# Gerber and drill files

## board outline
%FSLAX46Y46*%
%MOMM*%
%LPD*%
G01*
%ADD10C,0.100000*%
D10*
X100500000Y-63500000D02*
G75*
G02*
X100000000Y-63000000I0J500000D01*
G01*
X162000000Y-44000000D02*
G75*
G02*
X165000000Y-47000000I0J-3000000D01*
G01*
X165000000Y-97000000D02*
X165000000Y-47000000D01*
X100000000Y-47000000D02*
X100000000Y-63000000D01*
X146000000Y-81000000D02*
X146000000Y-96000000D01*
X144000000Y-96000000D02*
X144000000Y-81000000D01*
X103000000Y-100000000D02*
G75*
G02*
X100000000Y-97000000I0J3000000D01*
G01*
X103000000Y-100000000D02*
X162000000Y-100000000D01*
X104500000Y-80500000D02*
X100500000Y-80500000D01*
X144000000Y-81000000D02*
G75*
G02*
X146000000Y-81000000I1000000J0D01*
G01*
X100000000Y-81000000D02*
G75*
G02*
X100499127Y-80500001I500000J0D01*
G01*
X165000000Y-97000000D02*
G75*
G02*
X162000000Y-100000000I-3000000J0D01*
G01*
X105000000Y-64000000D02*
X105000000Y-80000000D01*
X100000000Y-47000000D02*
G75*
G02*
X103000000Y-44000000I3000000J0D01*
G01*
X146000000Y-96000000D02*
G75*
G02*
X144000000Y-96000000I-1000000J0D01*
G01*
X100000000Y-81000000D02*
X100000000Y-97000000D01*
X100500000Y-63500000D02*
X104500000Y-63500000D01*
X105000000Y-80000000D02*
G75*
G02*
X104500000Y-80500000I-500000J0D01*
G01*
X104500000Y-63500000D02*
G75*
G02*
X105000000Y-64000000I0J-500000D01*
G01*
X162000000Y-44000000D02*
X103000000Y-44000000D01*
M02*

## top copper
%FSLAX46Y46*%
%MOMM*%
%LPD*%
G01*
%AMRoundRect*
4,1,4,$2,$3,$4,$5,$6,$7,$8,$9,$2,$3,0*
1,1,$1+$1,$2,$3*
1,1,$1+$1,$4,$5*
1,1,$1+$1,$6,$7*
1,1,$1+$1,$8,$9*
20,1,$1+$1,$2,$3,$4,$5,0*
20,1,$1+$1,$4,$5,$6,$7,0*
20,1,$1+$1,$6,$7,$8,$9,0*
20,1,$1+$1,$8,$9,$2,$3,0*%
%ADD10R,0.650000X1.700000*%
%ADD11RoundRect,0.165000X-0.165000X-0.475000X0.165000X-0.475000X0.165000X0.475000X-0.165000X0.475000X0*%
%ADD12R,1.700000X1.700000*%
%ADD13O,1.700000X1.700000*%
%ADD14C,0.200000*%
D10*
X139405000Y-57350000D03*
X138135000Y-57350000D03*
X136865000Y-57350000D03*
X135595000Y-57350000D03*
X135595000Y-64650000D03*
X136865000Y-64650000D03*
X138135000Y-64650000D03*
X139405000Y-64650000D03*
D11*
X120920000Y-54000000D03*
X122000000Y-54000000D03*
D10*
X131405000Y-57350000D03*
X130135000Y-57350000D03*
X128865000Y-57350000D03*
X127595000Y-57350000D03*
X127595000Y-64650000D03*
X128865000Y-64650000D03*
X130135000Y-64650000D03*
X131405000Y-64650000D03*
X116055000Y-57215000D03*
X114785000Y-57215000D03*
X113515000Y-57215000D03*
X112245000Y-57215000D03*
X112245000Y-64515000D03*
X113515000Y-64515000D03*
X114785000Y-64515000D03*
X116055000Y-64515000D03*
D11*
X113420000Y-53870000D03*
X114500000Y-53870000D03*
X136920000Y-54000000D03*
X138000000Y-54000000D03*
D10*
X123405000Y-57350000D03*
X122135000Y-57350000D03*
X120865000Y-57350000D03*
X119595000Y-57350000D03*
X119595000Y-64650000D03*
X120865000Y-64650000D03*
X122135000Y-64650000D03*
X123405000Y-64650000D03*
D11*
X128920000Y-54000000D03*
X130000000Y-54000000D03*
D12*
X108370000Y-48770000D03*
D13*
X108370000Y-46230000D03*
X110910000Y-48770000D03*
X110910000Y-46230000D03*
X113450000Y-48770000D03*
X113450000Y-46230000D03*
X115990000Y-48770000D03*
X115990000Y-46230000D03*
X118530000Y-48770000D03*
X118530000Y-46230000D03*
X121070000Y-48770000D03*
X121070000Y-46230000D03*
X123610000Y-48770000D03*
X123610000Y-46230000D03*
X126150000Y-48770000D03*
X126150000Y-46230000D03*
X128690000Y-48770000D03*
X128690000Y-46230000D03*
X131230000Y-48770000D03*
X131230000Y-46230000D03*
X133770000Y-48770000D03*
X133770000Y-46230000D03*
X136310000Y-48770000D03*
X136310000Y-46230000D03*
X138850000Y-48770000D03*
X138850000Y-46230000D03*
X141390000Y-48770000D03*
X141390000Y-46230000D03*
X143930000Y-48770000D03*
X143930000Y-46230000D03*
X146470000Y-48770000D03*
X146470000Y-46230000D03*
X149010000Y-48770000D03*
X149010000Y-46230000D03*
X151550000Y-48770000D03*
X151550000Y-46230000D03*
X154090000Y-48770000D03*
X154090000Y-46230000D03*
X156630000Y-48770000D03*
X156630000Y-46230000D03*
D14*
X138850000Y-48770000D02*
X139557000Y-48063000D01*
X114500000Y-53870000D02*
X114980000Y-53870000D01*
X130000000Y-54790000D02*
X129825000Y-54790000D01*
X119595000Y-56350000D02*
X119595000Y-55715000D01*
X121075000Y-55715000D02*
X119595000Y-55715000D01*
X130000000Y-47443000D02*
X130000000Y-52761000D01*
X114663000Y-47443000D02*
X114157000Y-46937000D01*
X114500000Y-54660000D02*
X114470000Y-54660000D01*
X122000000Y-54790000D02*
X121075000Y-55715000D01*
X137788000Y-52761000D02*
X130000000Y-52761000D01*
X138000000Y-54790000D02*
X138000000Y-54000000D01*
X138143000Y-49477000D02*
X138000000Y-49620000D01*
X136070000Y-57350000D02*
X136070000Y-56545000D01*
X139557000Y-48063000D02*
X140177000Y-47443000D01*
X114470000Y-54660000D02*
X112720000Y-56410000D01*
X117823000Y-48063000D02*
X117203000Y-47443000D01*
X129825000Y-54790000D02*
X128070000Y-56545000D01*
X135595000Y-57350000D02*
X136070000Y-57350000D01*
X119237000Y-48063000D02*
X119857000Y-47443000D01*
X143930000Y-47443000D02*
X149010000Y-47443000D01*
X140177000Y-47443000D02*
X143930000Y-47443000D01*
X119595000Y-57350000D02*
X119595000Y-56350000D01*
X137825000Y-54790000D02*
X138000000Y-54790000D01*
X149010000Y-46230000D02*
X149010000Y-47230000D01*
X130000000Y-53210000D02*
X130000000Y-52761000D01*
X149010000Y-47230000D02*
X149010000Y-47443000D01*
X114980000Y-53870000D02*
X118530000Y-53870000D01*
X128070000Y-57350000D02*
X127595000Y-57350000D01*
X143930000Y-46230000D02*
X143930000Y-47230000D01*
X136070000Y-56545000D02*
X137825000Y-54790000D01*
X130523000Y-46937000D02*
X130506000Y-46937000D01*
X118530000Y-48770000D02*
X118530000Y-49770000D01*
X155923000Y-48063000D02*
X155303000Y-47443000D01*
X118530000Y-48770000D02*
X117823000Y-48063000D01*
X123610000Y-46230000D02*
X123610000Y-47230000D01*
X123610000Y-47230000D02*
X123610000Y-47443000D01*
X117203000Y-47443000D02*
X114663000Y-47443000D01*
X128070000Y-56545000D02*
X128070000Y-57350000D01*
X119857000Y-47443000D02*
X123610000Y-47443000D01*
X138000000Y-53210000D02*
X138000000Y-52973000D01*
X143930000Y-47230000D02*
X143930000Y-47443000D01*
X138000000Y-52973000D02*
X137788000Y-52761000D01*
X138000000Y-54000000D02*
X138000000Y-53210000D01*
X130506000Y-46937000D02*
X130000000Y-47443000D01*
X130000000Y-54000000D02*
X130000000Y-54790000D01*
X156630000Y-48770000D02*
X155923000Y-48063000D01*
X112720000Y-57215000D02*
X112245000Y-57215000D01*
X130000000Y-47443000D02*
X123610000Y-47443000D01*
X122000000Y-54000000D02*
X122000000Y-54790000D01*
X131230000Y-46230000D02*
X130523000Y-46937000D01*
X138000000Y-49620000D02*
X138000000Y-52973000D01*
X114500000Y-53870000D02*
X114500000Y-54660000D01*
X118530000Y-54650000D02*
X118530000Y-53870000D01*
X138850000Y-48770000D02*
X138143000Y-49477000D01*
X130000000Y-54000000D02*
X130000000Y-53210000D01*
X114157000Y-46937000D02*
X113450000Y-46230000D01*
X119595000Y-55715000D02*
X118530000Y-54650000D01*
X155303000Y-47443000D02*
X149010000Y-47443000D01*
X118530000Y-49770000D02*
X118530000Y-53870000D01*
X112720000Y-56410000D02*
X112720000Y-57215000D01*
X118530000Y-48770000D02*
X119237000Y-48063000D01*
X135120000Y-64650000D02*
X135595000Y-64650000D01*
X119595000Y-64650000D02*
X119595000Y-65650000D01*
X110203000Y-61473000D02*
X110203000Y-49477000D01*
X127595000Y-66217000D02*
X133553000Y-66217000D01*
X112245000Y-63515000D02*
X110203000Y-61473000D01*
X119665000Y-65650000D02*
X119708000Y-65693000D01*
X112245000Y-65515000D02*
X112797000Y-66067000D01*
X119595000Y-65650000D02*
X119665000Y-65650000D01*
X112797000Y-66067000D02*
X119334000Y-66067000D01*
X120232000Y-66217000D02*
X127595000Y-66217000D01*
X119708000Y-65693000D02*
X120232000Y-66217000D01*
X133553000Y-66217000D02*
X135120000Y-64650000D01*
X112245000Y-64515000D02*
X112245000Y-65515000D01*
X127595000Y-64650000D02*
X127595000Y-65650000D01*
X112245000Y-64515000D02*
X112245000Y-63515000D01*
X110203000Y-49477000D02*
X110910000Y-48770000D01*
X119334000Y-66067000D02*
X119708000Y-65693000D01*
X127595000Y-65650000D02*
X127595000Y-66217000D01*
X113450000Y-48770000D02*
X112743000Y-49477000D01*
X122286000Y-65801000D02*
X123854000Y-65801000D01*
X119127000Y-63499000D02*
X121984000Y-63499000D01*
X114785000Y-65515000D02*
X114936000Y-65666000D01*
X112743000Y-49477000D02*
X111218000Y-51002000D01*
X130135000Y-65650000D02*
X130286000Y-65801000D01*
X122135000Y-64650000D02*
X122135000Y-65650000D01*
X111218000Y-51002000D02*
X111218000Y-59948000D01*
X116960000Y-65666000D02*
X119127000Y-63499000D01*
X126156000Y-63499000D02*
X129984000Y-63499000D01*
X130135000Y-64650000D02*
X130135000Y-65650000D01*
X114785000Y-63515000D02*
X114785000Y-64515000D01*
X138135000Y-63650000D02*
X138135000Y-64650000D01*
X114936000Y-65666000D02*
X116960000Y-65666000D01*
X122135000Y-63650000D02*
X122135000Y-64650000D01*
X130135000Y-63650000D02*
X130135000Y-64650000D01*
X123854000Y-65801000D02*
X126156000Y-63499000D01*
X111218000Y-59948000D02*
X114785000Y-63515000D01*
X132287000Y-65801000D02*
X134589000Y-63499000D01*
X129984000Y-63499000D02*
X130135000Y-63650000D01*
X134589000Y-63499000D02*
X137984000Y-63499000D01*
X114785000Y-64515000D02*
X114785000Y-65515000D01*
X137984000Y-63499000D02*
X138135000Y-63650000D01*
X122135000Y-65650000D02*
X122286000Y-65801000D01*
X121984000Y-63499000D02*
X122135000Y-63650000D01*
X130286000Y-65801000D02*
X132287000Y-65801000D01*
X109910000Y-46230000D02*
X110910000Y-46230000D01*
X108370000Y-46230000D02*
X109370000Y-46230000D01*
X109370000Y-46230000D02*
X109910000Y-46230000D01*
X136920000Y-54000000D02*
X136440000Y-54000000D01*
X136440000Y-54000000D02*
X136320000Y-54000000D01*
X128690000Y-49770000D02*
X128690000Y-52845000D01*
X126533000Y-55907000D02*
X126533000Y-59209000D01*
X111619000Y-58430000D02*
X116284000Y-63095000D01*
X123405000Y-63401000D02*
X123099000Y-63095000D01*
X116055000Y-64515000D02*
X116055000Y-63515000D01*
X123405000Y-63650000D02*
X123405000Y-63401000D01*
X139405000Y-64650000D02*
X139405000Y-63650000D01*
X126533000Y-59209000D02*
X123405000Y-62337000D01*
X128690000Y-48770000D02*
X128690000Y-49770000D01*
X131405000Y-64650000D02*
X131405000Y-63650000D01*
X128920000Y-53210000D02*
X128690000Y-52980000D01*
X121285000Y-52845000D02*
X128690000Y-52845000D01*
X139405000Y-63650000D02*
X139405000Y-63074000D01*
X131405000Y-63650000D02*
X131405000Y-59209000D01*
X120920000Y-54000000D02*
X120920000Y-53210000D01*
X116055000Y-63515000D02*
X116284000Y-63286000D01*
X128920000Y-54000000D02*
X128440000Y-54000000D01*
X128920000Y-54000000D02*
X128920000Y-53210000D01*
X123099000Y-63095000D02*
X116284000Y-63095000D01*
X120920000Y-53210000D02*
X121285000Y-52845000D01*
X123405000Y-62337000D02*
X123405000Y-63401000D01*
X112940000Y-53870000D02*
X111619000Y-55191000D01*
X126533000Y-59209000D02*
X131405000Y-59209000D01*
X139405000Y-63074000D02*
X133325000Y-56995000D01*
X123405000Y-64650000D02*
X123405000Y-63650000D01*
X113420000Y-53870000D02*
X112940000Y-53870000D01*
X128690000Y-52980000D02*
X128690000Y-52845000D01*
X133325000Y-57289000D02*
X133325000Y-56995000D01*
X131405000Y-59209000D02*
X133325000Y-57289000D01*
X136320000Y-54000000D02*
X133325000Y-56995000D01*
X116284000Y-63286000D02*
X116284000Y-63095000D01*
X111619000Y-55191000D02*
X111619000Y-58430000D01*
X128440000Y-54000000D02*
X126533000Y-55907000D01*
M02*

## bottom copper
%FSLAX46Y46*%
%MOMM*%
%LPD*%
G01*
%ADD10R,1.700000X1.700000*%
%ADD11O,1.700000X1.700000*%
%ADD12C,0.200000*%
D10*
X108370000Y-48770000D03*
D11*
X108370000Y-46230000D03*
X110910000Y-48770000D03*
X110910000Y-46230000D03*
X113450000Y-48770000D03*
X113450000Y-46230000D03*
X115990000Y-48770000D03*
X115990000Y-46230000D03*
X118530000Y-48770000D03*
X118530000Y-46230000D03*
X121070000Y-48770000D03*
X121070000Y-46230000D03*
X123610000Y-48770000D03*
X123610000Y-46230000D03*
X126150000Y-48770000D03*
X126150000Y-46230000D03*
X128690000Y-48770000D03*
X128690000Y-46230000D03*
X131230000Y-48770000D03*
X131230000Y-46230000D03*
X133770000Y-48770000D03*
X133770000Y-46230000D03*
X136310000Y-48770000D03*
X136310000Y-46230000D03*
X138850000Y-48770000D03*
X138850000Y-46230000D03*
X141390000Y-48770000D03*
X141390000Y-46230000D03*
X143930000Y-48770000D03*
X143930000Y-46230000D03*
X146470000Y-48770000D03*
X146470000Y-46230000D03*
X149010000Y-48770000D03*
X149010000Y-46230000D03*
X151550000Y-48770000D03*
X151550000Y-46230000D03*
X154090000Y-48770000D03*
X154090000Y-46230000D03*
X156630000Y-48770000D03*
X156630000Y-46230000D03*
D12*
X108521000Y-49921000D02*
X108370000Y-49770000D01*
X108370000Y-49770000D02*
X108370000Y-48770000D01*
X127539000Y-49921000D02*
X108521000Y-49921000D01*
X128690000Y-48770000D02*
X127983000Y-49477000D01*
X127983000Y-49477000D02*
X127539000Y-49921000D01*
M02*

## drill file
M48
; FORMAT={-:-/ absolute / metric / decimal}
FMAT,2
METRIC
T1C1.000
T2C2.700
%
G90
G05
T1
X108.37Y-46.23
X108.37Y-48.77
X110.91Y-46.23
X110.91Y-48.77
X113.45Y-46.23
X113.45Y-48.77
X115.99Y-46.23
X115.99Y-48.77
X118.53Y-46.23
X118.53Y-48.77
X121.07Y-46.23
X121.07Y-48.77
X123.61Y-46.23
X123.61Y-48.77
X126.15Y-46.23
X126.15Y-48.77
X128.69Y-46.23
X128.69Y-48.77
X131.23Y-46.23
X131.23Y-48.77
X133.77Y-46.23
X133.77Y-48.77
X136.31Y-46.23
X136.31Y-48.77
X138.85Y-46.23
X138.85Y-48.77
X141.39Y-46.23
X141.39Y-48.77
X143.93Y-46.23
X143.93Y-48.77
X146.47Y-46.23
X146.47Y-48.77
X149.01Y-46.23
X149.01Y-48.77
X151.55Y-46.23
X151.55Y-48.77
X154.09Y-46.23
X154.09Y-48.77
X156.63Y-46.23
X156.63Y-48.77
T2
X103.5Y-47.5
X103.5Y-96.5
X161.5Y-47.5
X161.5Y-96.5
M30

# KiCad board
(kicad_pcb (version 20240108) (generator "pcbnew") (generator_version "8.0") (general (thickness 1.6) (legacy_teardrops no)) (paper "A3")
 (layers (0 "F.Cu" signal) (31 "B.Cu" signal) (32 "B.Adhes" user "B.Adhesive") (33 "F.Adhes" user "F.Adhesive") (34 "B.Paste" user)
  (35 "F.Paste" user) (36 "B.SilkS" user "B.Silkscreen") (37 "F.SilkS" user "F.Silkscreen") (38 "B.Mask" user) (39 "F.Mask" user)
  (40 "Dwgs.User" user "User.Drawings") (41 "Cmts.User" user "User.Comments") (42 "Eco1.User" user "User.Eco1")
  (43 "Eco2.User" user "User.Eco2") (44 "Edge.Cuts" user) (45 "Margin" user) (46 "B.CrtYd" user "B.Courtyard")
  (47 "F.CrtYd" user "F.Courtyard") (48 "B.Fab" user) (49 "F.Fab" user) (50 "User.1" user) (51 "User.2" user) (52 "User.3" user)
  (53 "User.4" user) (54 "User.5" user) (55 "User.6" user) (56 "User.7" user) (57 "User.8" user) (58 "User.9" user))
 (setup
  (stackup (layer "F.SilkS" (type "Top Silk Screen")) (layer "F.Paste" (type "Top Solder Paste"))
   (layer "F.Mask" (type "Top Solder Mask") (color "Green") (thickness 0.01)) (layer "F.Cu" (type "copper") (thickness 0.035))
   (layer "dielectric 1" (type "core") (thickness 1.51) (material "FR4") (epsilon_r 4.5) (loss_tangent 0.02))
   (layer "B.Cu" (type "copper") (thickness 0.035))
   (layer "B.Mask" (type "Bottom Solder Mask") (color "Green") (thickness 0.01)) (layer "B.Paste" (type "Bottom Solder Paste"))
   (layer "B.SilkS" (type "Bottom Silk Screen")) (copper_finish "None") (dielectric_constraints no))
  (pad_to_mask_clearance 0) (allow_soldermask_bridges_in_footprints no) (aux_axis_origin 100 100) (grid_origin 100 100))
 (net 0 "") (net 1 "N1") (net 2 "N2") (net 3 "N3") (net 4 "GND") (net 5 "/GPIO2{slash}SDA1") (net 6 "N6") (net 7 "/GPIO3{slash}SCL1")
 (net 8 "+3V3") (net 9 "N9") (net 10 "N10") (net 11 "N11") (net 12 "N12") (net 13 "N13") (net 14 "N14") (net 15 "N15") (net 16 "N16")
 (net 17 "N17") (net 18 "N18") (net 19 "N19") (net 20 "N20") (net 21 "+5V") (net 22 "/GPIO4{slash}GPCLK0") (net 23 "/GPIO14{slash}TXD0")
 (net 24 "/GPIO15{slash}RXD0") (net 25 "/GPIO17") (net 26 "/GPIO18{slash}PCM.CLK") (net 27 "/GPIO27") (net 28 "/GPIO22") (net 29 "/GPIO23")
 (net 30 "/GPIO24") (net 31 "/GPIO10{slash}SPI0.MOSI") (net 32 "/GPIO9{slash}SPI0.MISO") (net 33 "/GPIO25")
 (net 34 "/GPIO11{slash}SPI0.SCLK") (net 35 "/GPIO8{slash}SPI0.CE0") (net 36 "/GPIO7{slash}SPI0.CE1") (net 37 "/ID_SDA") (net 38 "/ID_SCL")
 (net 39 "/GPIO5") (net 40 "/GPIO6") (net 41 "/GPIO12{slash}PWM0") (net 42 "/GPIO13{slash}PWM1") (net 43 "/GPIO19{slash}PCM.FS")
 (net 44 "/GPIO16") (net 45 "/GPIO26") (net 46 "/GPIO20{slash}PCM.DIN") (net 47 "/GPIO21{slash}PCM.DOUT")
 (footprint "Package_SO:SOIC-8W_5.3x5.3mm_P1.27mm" (layer "F.Cu") (at 137.5 61 -90)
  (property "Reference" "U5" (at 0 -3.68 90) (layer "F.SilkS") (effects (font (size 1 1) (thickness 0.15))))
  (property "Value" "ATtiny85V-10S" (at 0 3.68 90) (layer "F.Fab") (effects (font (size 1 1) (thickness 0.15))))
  (pad "1" smd rect (at -3.65 -1.905 270) (size 1.7 0.65) (layers "F.Cu" "F.Paste" "F.Mask") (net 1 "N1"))
  (pad "2" smd rect (at -3.65 -0.635 270) (size 1.7 0.65) (layers "F.Cu" "F.Paste" "F.Mask") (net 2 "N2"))
  (pad "3" smd rect (at -3.65 0.635 270) (size 1.7 0.65) (layers "F.Cu" "F.Paste" "F.Mask") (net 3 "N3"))
  (pad "4" smd rect (at -3.65 1.905 270) (size 1.7 0.65) (layers "F.Cu" "F.Paste" "F.Mask") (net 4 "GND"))
  (pad "5" smd rect (at 3.65 1.905 270) (size 1.7 0.65) (layers "F.Cu" "F.Paste" "F.Mask") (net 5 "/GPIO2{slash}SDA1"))
  (pad "6" smd rect (at 3.65 0.635 270) (size 1.7 0.65) (layers "F.Cu" "F.Paste" "F.Mask") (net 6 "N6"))
  (pad "7" smd rect (at 3.65 -0.635 270) (size 1.7 0.65) (layers "F.Cu" "F.Paste" "F.Mask") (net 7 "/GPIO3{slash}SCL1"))
  (pad "8" smd rect (at 3.65 -1.905 270) (size 1.7 0.65) (layers "F.Cu" "F.Paste" "F.Mask") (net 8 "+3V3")))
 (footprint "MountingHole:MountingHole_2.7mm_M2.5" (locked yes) (layer "F.Cu") (at 161.5 47.5)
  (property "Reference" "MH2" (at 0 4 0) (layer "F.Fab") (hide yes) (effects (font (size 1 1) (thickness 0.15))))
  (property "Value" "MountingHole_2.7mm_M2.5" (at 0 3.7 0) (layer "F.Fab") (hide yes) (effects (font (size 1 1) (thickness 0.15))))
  (pad "" np_thru_hole circle (at 0 0) (size 2.7 2.7) (drill 2.7) (layers "*.Cu" "*.Mask")))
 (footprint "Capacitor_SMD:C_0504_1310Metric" (layer "F.Cu") (at 121.46 54)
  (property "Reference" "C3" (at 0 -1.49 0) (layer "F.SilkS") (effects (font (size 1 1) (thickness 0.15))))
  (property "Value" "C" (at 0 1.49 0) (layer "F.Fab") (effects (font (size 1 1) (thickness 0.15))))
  (pad "1" smd roundrect (at -0.54 0) (size 0.66 1.28) (layers "F.Cu" "F.Paste" "F.Mask") (roundrect_rratio 0.25) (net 8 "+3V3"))
  (pad "2" smd roundrect (at 0.54 0) (size 0.66 1.28) (layers "F.Cu" "F.Paste" "F.Mask") (roundrect_rratio 0.25) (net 4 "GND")))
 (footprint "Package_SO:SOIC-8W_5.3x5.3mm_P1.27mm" (layer "F.Cu") (at 129.5 61 -90)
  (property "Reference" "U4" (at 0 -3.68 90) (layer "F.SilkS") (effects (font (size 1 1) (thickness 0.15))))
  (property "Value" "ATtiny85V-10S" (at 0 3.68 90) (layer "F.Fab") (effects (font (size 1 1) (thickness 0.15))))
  (pad "1" smd rect (at -3.65 -1.905 270) (size 1.7 0.65) (layers "F.Cu" "F.Paste" "F.Mask") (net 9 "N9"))
  (pad "2" smd rect (at -3.65 -0.635 270) (size 1.7 0.65) (layers "F.Cu" "F.Paste" "F.Mask") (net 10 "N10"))
  (pad "3" smd rect (at -3.65 0.635 270) (size 1.7 0.65) (layers "F.Cu" "F.Paste" "F.Mask") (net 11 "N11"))
  (pad "4" smd rect (at -3.65 1.905 270) (size 1.7 0.65) (layers "F.Cu" "F.Paste" "F.Mask") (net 4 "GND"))
  (pad "5" smd rect (at 3.65 1.905 270) (size 1.7 0.65) (layers "F.Cu" "F.Paste" "F.Mask") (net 5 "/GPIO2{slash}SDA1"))
  (pad "6" smd rect (at 3.65 0.635 270) (size 1.7 0.65) (layers "F.Cu" "F.Paste" "F.Mask") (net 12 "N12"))
  (pad "7" smd rect (at 3.65 -0.635 270) (size 1.7 0.65) (layers "F.Cu" "F.Paste" "F.Mask") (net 7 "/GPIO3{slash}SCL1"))
  (pad "8" smd rect (at 3.65 -1.905 270) (size 1.7 0.65) (layers "F.Cu" "F.Paste" "F.Mask") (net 8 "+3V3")))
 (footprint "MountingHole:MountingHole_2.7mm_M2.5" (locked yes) (layer "F.Cu") (at 103.5 96.5)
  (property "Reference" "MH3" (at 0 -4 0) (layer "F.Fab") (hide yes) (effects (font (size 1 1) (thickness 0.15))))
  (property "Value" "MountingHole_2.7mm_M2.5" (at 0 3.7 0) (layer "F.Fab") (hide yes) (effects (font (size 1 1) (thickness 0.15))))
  (pad "" np_thru_hole circle (at 0 0) (size 2.7 2.7) (drill 2.7) (layers "*.Cu" "*.Mask")))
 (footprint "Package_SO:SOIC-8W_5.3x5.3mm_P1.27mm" (layer "F.Cu") (at 114.15 60.865 -90)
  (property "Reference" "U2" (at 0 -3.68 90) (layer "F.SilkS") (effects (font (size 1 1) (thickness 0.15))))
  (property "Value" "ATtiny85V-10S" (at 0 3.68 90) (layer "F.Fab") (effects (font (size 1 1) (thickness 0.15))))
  (pad "1" smd rect (at -3.65 -1.905 270) (size 1.7 0.65) (layers "F.Cu" "F.Paste" "F.Mask") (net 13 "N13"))
  (pad "2" smd rect (at -3.65 -0.635 270) (size 1.7 0.65) (layers "F.Cu" "F.Paste" "F.Mask") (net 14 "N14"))
  (pad "3" smd rect (at -3.65 0.635 270) (size 1.7 0.65) (layers "F.Cu" "F.Paste" "F.Mask") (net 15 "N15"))
  (pad "4" smd rect (at -3.65 1.905 270) (size 1.7 0.65) (layers "F.Cu" "F.Paste" "F.Mask") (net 4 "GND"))
  (pad "5" smd rect (at 3.65 1.905 270) (size 1.7 0.65) (layers "F.Cu" "F.Paste" "F.Mask") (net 5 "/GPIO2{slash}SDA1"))
  (pad "6" smd rect (at 3.65 0.635 270) (size 1.7 0.65) (layers "F.Cu" "F.Paste" "F.Mask") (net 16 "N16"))
  (pad "7" smd rect (at 3.65 -0.635 270) (size 1.7 0.65) (layers "F.Cu" "F.Paste" "F.Mask") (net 7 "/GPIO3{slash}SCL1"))
  (pad "8" smd rect (at 3.65 -1.905 270) (size 1.7 0.65) (layers "F.Cu" "F.Paste" "F.Mask") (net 8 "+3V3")))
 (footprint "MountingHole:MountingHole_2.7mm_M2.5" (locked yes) (layer "F.Cu") (at 103.5 47.5)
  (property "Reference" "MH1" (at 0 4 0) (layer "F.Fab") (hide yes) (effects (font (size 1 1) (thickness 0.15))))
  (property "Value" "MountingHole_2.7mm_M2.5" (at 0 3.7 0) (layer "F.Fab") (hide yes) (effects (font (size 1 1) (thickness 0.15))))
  (pad "" np_thru_hole circle (at 0 0) (size 2.7 2.7) (drill 2.7) (layers "*.Cu" "*.Mask")))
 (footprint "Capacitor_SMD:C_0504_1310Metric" (layer "F.Cu") (at 113.96 53.87)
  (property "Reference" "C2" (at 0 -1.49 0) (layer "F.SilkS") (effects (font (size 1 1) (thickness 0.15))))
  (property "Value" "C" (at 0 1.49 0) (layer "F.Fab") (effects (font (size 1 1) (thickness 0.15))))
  (pad "1" smd roundrect (at -0.54 0) (size 0.66 1.28) (layers "F.Cu" "F.Paste" "F.Mask") (roundrect_rratio 0.25) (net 8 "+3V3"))
  (pad "2" smd roundrect (at 0.54 0) (size 0.66 1.28) (layers "F.Cu" "F.Paste" "F.Mask") (roundrect_rratio 0.25) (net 4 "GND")))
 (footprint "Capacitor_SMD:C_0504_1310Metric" (layer "F.Cu") (at 137.46 54)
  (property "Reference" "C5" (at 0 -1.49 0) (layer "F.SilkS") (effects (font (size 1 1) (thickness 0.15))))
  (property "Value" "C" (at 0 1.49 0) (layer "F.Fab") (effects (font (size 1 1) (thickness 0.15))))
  (pad "1" smd roundrect (at -0.54 0) (size 0.66 1.28) (layers "F.Cu" "F.Paste" "F.Mask") (roundrect_rratio 0.25) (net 8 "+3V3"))
  (pad "2" smd roundrect (at 0.54 0) (size 0.66 1.28) (layers "F.Cu" "F.Paste" "F.Mask") (roundrect_rratio 0.25) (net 4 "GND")))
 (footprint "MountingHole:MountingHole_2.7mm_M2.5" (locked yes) (layer "F.Cu") (at 161.5 96.5)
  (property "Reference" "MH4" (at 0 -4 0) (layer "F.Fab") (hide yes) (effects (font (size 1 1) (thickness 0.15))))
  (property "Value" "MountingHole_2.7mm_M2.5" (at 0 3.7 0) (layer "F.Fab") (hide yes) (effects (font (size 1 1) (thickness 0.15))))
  (pad "" np_thru_hole circle (at 0 0) (size 2.7 2.7) (drill 2.7) (layers "*.Cu" "*.Mask")))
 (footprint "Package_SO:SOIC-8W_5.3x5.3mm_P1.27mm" (layer "F.Cu") (at 121.5 61 -90)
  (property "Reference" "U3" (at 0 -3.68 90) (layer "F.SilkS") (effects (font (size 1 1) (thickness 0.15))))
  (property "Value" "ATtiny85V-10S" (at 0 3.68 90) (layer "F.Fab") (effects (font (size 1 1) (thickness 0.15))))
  (pad "1" smd rect (at -3.65 -1.905 270) (size 1.7 0.65) (layers "F.Cu" "F.Paste" "F.Mask") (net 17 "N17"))
  (pad "2" smd rect (at -3.65 -0.635 270) (size 1.7 0.65) (layers "F.Cu" "F.Paste" "F.Mask") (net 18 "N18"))
  (pad "3" smd rect (at -3.65 0.635 270) (size 1.7 0.65) (layers "F.Cu" "F.Paste" "F.Mask") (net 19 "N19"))
  (pad "4" smd rect (at -3.65 1.905 270) (size 1.7 0.65) (layers "F.Cu" "F.Paste" "F.Mask") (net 4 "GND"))
  (pad "5" smd rect (at 3.65 1.905 270) (size 1.7 0.65) (layers "F.Cu" "F.Paste" "F.Mask") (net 5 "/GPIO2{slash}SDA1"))
  (pad "6" smd rect (at 3.65 0.635 270) (size 1.7 0.65) (layers "F.Cu" "F.Paste" "F.Mask") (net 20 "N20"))
  (pad "7" smd rect (at 3.65 -0.635 270) (size 1.7 0.65) (layers "F.Cu" "F.Paste" "F.Mask") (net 7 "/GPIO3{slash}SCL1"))
  (pad "8" smd rect (at 3.65 -1.905 270) (size 1.7 0.65) (layers "F.Cu" "F.Paste" "F.Mask") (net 8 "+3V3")))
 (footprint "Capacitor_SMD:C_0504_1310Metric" (layer "F.Cu") (at 129.46 54)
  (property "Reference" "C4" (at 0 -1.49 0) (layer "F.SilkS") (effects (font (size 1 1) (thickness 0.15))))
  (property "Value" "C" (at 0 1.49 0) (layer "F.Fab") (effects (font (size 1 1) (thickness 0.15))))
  (pad "1" smd roundrect (at -0.54 0) (size 0.66 1.28) (layers "F.Cu" "F.Paste" "F.Mask") (roundrect_rratio 0.25) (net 8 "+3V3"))
  (pad "2" smd roundrect (at 0.54 0) (size 0.66 1.28) (layers "F.Cu" "F.Paste" "F.Mask") (roundrect_rratio 0.25) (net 4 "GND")))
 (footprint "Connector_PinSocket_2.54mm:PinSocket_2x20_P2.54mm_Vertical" (layer "B.Cu") (at 108.37 48.77 -90)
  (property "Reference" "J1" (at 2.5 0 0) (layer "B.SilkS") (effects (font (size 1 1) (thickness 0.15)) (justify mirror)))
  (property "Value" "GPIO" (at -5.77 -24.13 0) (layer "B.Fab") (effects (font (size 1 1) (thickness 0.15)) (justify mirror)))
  (pad "1" thru_hole rect (at 0 0 270) (size 1.7 1.7) (drill 1) (layers "*.Cu" "*.Mask") (remove_unused_layers no) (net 8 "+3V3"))
  (pad "2" thru_hole oval (at -2.54 0 270) (size 1.7 1.7) (drill 1) (layers "*.Cu" "*.Mask") (remove_unused_layers no) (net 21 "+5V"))
  (pad "3" thru_hole oval (at 0 -2.54 270) (size 1.7 1.7) (drill 1) (layers "*.Cu" "*.Mask") (remove_unused_layers no)
   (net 5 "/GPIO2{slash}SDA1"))
  (pad "4" thru_hole oval (at -2.54 -2.54 270) (size 1.7 1.7) (drill 1) (layers "*.Cu" "*.Mask") (remove_unused_layers no) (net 21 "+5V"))
  (pad "5" thru_hole oval (at 0 -5.08 270) (size 1.7 1.7) (drill 1) (layers "*.Cu" "*.Mask") (remove_unused_layers no)
   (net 7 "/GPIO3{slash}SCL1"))
  (pad "6" thru_hole oval (at -2.54 -5.08 270) (size 1.7 1.7) (drill 1) (layers "*.Cu" "*.Mask") (remove_unused_layers no) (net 4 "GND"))
  (pad "7" thru_hole oval (at 0 -7.62 270) (size 1.7 1.7) (drill 1) (layers "*.Cu" "*.Mask") (remove_unused_layers no)
   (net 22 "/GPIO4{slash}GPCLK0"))
  (pad "8" thru_hole oval (at -2.54 -7.62 270) (size 1.7 1.7) (drill 1) (layers "*.Cu" "*.Mask") (remove_unused_layers no)
   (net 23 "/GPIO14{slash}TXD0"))
  (pad "9" thru_hole oval (at 0 -10.16 270) (size 1.7 1.7) (drill 1) (layers "*.Cu" "*.Mask") (remove_unused_layers no) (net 4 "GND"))
  (pad "10" thru_hole oval (at -2.54 -10.16 270) (size 1.7 1.7) (drill 1) (layers "*.Cu" "*.Mask") (remove_unused_layers no)
   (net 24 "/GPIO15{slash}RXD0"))
  (pad "11" thru_hole oval (at 0 -12.7 270) (size 1.7 1.7) (drill 1) (layers "*.Cu" "*.Mask") (remove_unused_layers no) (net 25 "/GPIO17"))
  (pad "12" thru_hole oval (at -2.54 -12.7 270) (size 1.7 1.7) (drill 1) (layers "*.Cu" "*.Mask") (remove_unused_layers no)
   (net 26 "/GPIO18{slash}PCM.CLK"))
  (pad "13" thru_hole oval (at 0 -15.24 270) (size 1.7 1.7) (drill 1) (layers "*.Cu" "*.Mask") (remove_unused_layers no) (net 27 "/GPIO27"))
  (pad "14" thru_hole oval (at -2.54 -15.24 270) (size 1.7 1.7) (drill 1) (layers "*.Cu" "*.Mask") (remove_unused_layers no) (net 4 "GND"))
  (pad "15" thru_hole oval (at 0 -17.78 270) (size 1.7 1.7) (drill 1) (layers "*.Cu" "*.Mask") (remove_unused_layers no) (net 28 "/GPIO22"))
  (pad "16" thru_hole oval (at -2.54 -17.78 270) (size 1.7 1.7) (drill 1) (layers "*.Cu" "*.Mask") (remove_unused_layers no)
   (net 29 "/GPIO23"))
  (pad "17" thru_hole oval (at 0 -20.32 270) (size 1.7 1.7) (drill 1) (layers "*.Cu" "*.Mask") (remove_unused_layers no) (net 8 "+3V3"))
  (pad "18" thru_hole oval (at -2.54 -20.32 270) (size 1.7 1.7) (drill 1) (layers "*.Cu" "*.Mask") (remove_unused_layers no)
   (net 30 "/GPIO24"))
  (pad "19" thru_hole oval (at 0 -22.86 270) (size 1.7 1.7) (drill 1) (layers "*.Cu" "*.Mask") (remove_unused_layers no)
   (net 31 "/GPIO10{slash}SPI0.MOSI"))
  (pad "20" thru_hole oval (at -2.54 -22.86 270) (size 1.7 1.7) (drill 1) (layers "*.Cu" "*.Mask") (remove_unused_layers no) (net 4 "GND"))
  (pad "21" thru_hole oval (at 0 -25.4 270) (size 1.7 1.7) (drill 1) (layers "*.Cu" "*.Mask") (remove_unused_layers no)
   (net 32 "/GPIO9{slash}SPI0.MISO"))
  (pad "22" thru_hole oval (at -2.54 -25.4 270) (size 1.7 1.7) (drill 1) (layers "*.Cu" "*.Mask") (remove_unused_layers no)
   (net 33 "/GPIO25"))
  (pad "23" thru_hole oval (at 0 -27.94 270) (size 1.7 1.7) (drill 1) (layers "*.Cu" "*.Mask") (remove_unused_layers no)
   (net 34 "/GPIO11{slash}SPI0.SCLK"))
  (pad "24" thru_hole oval (at -2.54 -27.94 270) (size 1.7 1.7) (drill 1) (layers "*.Cu" "*.Mask") (remove_unused_layers no)
   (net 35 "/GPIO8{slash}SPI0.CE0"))
  (pad "25" thru_hole oval (at 0 -30.48 270) (size 1.7 1.7) (drill 1) (layers "*.Cu" "*.Mask") (remove_unused_layers no) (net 4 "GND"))
  (pad "26" thru_hole oval (at -2.54 -30.48 270) (size 1.7 1.7) (drill 1) (layers "*.Cu" "*.Mask") (remove_unused_layers no)
   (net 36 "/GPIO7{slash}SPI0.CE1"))
  (pad "27" thru_hole oval (at 0 -33.02 270) (size 1.7 1.7) (drill 1) (layers "*.Cu" "*.Mask") (remove_unused_layers no) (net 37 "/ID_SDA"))
  (pad "28" thru_hole oval (at -2.54 -33.02 270) (size 1.7 1.7) (drill 1) (layers "*.Cu" "*.Mask") (remove_unused_layers no)
   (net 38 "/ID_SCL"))
  (pad "29" thru_hole oval (at 0 -35.56 270) (size 1.7 1.7) (drill 1) (layers "*.Cu" "*.Mask") (remove_unused_layers no) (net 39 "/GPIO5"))
  (pad "30" thru_hole oval (at -2.54 -35.56 270) (size 1.7 1.7) (drill 1) (layers "*.Cu" "*.Mask") (remove_unused_layers no) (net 4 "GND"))
  (pad "31" thru_hole oval (at 0 -38.1 270) (size 1.7 1.7) (drill 1) (layers "*.Cu" "*.Mask") (remove_unused_layers no) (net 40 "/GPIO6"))
  (pad "32" thru_hole oval (at -2.54 -38.1 270) (size 1.7 1.7) (drill 1) (layers "*.Cu" "*.Mask") (remove_unused_layers no)
   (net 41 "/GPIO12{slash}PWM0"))
  (pad "33" thru_hole oval (at 0 -40.64 270) (size 1.7 1.7) (drill 1) (layers "*.Cu" "*.Mask") (remove_unused_layers no)
   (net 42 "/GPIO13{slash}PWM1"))
  (pad "34" thru_hole oval (at -2.54 -40.64 270) (size 1.7 1.7) (drill 1) (layers "*.Cu" "*.Mask") (remove_unused_layers no) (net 4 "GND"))
  (pad "35" thru_hole oval (at 0 -43.18 270) (size 1.7 1.7) (drill 1) (layers "*.Cu" "*.Mask") (remove_unused_layers no)
   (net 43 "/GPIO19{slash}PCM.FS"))
  (pad "36" thru_hole oval (at -2.54 -43.18 270) (size 1.7 1.7) (drill 1) (layers "*.Cu" "*.Mask") (remove_unused_layers no)
   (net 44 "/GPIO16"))
  (pad "37" thru_hole oval (at 0 -45.72 270) (size 1.7 1.7) (drill 1) (layers "*.Cu" "*.Mask") (remove_unused_layers no) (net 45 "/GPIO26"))
  (pad "38" thru_hole oval (at -2.54 -45.72 270) (size 1.7 1.7) (drill 1) (layers "*.Cu" "*.Mask") (remove_unused_layers no)
   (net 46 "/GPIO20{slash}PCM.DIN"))
  (pad "39" thru_hole oval (at 0 -48.26 270) (size 1.7 1.7) (drill 1) (layers "*.Cu" "*.Mask") (remove_unused_layers no) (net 4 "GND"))
  (pad "40" thru_hole oval (at -2.54 -48.26 270) (size 1.7 1.7) (drill 1) (layers "*.Cu" "*.Mask") (remove_unused_layers no)
   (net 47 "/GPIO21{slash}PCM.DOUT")))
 (gr_arc (start 100.5 63.5) (mid 100.146447 63.353553) (end 100 63) (stroke (width 0.1) (type solid)) (layer "Edge.Cuts"))
 (gr_arc (start 162 44) (mid 164.12132 44.87868) (end 165 47) (stroke (width 0.1) (type solid)) (layer "Edge.Cuts"))
 (gr_line (start 165 97) (end 165 47) (stroke (width 0.1) (type solid)) (layer "Edge.Cuts"))
 (gr_line (start 100 47) (end 100 63) (stroke (width 0.1) (type solid)) (layer "Edge.Cuts"))
 (gr_line (start 146 81) (end 146 96) (stroke (width 0.1) (type solid)) (layer "Edge.Cuts"))
 (gr_line (start 144 96) (end 144 81) (stroke (width 0.1) (type solid)) (layer "Edge.Cuts"))
 (gr_arc (start 103 100) (mid 100.87868 99.12132) (end 100 97) (stroke (width 0.1) (type solid)) (layer "Edge.Cuts"))
 (gr_line (start 103 100) (end 162 100) (stroke (width 0.1) (type solid)) (layer "Edge.Cuts"))
 (gr_line (start 104.5 80.5) (end 100.5 80.5) (stroke (width 0.1) (type solid)) (layer "Edge.Cuts"))
 (gr_arc (start 144 81) (mid 145 80) (end 146 81) (stroke (width 0.1) (type solid)) (layer "Edge.Cuts"))
 (gr_arc (start 100 81) (mid 100.146138 80.646755) (end 100.499127 80.500001) (stroke (width 0.1) (type solid)) (layer "Edge.Cuts"))
 (gr_arc (start 165 97) (mid 164.12132 99.12132) (end 162 100) (stroke (width 0.1) (type solid)) (layer "Edge.Cuts"))
 (gr_line (start 105 64) (end 105 80) (stroke (width 0.1) (type solid)) (layer "Edge.Cuts"))
 (gr_arc (start 100 47) (mid 100.87868 44.87868) (end 103 44) (stroke (width 0.1) (type solid)) (layer "Edge.Cuts"))
 (gr_arc (start 146 96) (mid 145 97) (end 144 96) (stroke (width 0.1) (type solid)) (layer "Edge.Cuts"))
 (gr_line (start 100 81) (end 100 97) (stroke (width 0.1) (type solid)) (layer "Edge.Cuts"))
 (gr_line (start 100.5 63.5) (end 104.5 63.5) (stroke (width 0.1) (type solid)) (layer "Edge.Cuts"))
 (gr_arc (start 105 80) (mid 104.853553 80.353553) (end 104.5 80.5) (stroke (width 0.1) (type solid)) (layer "Edge.Cuts"))
 (gr_arc (start 104.5 63.5) (mid 104.853553 63.646447) (end 105 64) (stroke (width 0.1) (type solid)) (layer "Edge.Cuts"))
 (gr_line (start 162 44) (end 103 44) (stroke (width 0.1) (type solid)) (layer "Edge.Cuts"))
 (segment (start 138.85 48.77) (end 139.557 48.063) (width 0.2) (layer "F.Cu") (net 4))
 (segment (start 114.5 53.87) (end 114.98 53.87) (width 0.2) (layer "F.Cu") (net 4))
 (segment (start 130 54.79) (end 129.825 54.79) (width 0.2) (layer "F.Cu") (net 4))
 (segment (start 119.595 56.35) (end 119.595 55.715) (width 0.2) (layer "F.Cu") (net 4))
 (segment (start 121.075 55.715) (end 119.595 55.715) (width 0.2) (layer "F.Cu") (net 4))
 (segment (start 130 47.443) (end 130 52.761) (width 0.2) (layer "F.Cu") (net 4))
 (segment (start 114.663 47.443) (end 114.157 46.937) (width 0.2) (layer "F.Cu") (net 4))
 (segment (start 114.5 54.66) (end 114.47 54.66) (width 0.2) (layer "F.Cu") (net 4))
 (segment (start 122 54.79) (end 121.075 55.715) (width 0.2) (layer "F.Cu") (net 4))
 (segment (start 137.788 52.761) (end 130 52.761) (width 0.2) (layer "F.Cu") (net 4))
 (segment (start 138 54.79) (end 138 54) (width 0.2) (layer "F.Cu") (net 4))
 (segment (start 138.143 49.477) (end 138 49.62) (width 0.2) (layer "F.Cu") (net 4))
 (segment (start 136.07 57.35) (end 136.07 56.545) (width 0.2) (layer "F.Cu") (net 4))
 (segment (start 139.557 48.063) (end 140.177 47.443) (width 0.2) (layer "F.Cu") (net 4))
 (segment (start 114.47 54.66) (end 112.72 56.41) (width 0.2) (layer "F.Cu") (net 4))
 (segment (start 117.823 48.063) (end 117.203 47.443) (width 0.2) (layer "F.Cu") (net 4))
 (segment (start 129.825 54.79) (end 128.07 56.545) (width 0.2) (layer "F.Cu") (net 4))
 (segment (start 135.595 57.35) (end 136.07 57.35) (width 0.2) (layer "F.Cu") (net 4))
 (segment (start 119.237 48.063) (end 119.857 47.443) (width 0.2) (layer "F.Cu") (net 4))
 (segment (start 143.93 47.443) (end 149.01 47.443) (width 0.2) (layer "F.Cu") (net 4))
 (segment (start 140.177 47.443) (end 143.93 47.443) (width 0.2) (layer "F.Cu") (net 4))
 (segment (start 119.595 57.35) (end 119.595 56.35) (width 0.2) (layer "F.Cu") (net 4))
 (segment (start 137.825 54.79) (end 138 54.79) (width 0.2) (layer "F.Cu") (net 4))
 (segment (start 149.01 46.23) (end 149.01 47.23) (width 0.2) (layer "F.Cu") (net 4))
 (segment (start 130 53.21) (end 130 52.761) (width 0.2) (layer "F.Cu") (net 4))
 (segment (start 149.01 47.23) (end 149.01 47.443) (width 0.2) (layer "F.Cu") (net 4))
 (segment (start 114.98 53.87) (end 118.53 53.87) (width 0.2) (layer "F.Cu") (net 4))
 (segment (start 128.07 57.35) (end 127.595 57.35) (width 0.2) (layer "F.Cu") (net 4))
 (segment (start 143.93 46.23) (end 143.93 47.23) (width 0.2) (layer "F.Cu") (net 4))
 (segment (start 136.07 56.545) (end 137.825 54.79) (width 0.2) (layer "F.Cu") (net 4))
 (segment (start 130.523 46.937) (end 130.506 46.937) (width 0.2) (layer "F.Cu") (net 4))
 (segment (start 118.53 48.77) (end 118.53 49.77) (width 0.2) (layer "F.Cu") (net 4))
 (segment (start 155.923 48.063) (end 155.303 47.443) (width 0.2) (layer "F.Cu") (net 4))
 (segment (start 118.53 48.77) (end 117.823 48.063) (width 0.2) (layer "F.Cu") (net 4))
 (segment (start 123.61 46.23) (end 123.61 47.23) (width 0.2) (layer "F.Cu") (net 4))
 (segment (start 123.61 47.23) (end 123.61 47.443) (width 0.2) (layer "F.Cu") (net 4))
 (segment (start 117.203 47.443) (end 114.663 47.443) (width 0.2) (layer "F.Cu") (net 4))
 (segment (start 128.07 56.545) (end 128.07 57.35) (width 0.2) (layer "F.Cu") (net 4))
 (segment (start 119.857 47.443) (end 123.61 47.443) (width 0.2) (layer "F.Cu") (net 4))
 (segment (start 138 53.21) (end 138 52.973) (width 0.2) (layer "F.Cu") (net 4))
 (segment (start 143.93 47.23) (end 143.93 47.443) (width 0.2) (layer "F.Cu") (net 4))
 (segment (start 138 52.973) (end 137.788 52.761) (width 0.2) (layer "F.Cu") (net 4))
 (segment (start 138 54) (end 138 53.21) (width 0.2) (layer "F.Cu") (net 4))
 (segment (start 130.506 46.937) (end 130 47.443) (width 0.2) (layer "F.Cu") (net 4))
 (segment (start 130 54) (end 130 54.79) (width 0.2) (layer "F.Cu") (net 4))
 (segment (start 156.63 48.77) (end 155.923 48.063) (width 0.2) (layer "F.Cu") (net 4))
 (segment (start 112.72 57.215) (end 112.245 57.215) (width 0.2) (layer "F.Cu") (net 4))
 (segment (start 130 47.443) (end 123.61 47.443) (width 0.2) (layer "F.Cu") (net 4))
 (segment (start 122 54) (end 122 54.79) (width 0.2) (layer "F.Cu") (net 4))
 (segment (start 131.23 46.23) (end 130.523 46.937) (width 0.2) (layer "F.Cu") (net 4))
 (segment (start 138 49.62) (end 138 52.973) (width 0.2) (layer "F.Cu") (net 4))
 (segment (start 114.5 53.87) (end 114.5 54.66) (width 0.2) (layer "F.Cu") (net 4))
 (segment (start 118.53 54.65) (end 118.53 53.87) (width 0.2) (layer "F.Cu") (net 4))
 (segment (start 138.85 48.77) (end 138.143 49.477) (width 0.2) (layer "F.Cu") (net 4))
 (segment (start 130 54) (end 130 53.21) (width 0.2) (layer "F.Cu") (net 4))
 (segment (start 114.157 46.937) (end 113.45 46.23) (width 0.2) (layer "F.Cu") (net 4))
 (segment (start 119.595 55.715) (end 118.53 54.65) (width 0.2) (layer "F.Cu") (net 4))
 (segment (start 155.303 47.443) (end 149.01 47.443) (width 0.2) (layer "F.Cu") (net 4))
 (segment (start 118.53 49.77) (end 118.53 53.87) (width 0.2) (layer "F.Cu") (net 4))
 (segment (start 112.72 56.41) (end 112.72 57.215) (width 0.2) (layer "F.Cu") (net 4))
 (segment (start 118.53 48.77) (end 119.237 48.063) (width 0.2) (layer "F.Cu") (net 4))
 (segment (start 135.12 64.65) (end 135.595 64.65) (width 0.2) (layer "F.Cu") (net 5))
 (segment (start 119.595 64.65) (end 119.595 65.65) (width 0.2) (layer "F.Cu") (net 5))
 (segment (start 110.203 61.473) (end 110.203 49.477) (width 0.2) (layer "F.Cu") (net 5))
 (segment (start 127.595 66.217) (end 133.553 66.217) (width 0.2) (layer "F.Cu") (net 5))
 (segment (start 112.245 63.515) (end 110.203 61.473) (width 0.2) (layer "F.Cu") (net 5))
 (segment (start 119.665 65.65) (end 119.708 65.693) (width 0.2) (layer "F.Cu") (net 5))
 (segment (start 112.245 65.515) (end 112.797 66.067) (width 0.2) (layer "F.Cu") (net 5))
 (segment (start 119.595 65.65) (end 119.665 65.65) (width 0.2) (layer "F.Cu") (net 5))
 (segment (start 112.797 66.067) (end 119.334 66.067) (width 0.2) (layer "F.Cu") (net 5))
 (segment (start 120.232 66.217) (end 127.595 66.217) (width 0.2) (layer "F.Cu") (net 5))
 (segment (start 119.708 65.693) (end 120.232 66.217) (width 0.2) (layer "F.Cu") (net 5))
 (segment (start 133.553 66.217) (end 135.12 64.65) (width 0.2) (layer "F.Cu") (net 5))
 (segment (start 112.245 64.515) (end 112.245 65.515) (width 0.2) (layer "F.Cu") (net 5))
 (segment (start 127.595 64.65) (end 127.595 65.65) (width 0.2) (layer "F.Cu") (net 5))
 (segment (start 112.245 64.515) (end 112.245 63.515) (width 0.2) (layer "F.Cu") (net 5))
 (segment (start 110.203 49.477) (end 110.91 48.77) (width 0.2) (layer "F.Cu") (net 5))
 (segment (start 119.334 66.067) (end 119.708 65.693) (width 0.2) (layer "F.Cu") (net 5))
 (segment (start 127.595 65.65) (end 127.595 66.217) (width 0.2) (layer "F.Cu") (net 5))
 (segment (start 113.45 48.77) (end 112.743 49.477) (width 0.2) (layer "F.Cu") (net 7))
 (segment (start 122.286 65.801) (end 123.854 65.801) (width 0.2) (layer "F.Cu") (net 7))
 (segment (start 119.127 63.499) (end 121.984 63.499) (width 0.2) (layer "F.Cu") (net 7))
 (segment (start 114.785 65.515) (end 114.936 65.666) (width 0.2) (layer "F.Cu") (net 7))
 (segment (start 112.743 49.477) (end 111.218 51.002) (width 0.2) (layer "F.Cu") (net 7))
 (segment (start 130.135 65.65) (end 130.286 65.801) (width 0.2) (layer "F.Cu") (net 7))
 (segment (start 122.135 64.65) (end 122.135 65.65) (width 0.2) (layer "F.Cu") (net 7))
 (segment (start 111.218 51.002) (end 111.218 59.948) (width 0.2) (layer "F.Cu") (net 7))
 (segment (start 116.96 65.666) (end 119.127 63.499) (width 0.2) (layer "F.Cu") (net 7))
 (segment (start 126.156 63.499) (end 129.984 63.499) (width 0.2) (layer "F.Cu") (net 7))
 (segment (start 130.135 64.65) (end 130.135 65.65) (width 0.2) (layer "F.Cu") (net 7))
 (segment (start 114.785 63.515) (end 114.785 64.515) (width 0.2) (layer "F.Cu") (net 7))
 (segment (start 138.135 63.65) (end 138.135 64.65) (width 0.2) (layer "F.Cu") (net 7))
 (segment (start 114.936 65.666) (end 116.96 65.666) (width 0.2) (layer "F.Cu") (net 7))
 (segment (start 122.135 63.65) (end 122.135 64.65) (width 0.2) (layer "F.Cu") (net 7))
 (segment (start 130.135 63.65) (end 130.135 64.65) (width 0.2) (layer "F.Cu") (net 7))
 (segment (start 123.854 65.801) (end 126.156 63.499) (width 0.2) (layer "F.Cu") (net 7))
 (segment (start 111.218 59.948) (end 114.785 63.515) (width 0.2) (layer "F.Cu") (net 7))
 (segment (start 132.287 65.801) (end 134.589 63.499) (width 0.2) (layer "F.Cu") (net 7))
 (segment (start 129.984 63.499) (end 130.135 63.65) (width 0.2) (layer "F.Cu") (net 7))
 (segment (start 134.589 63.499) (end 137.984 63.499) (width 0.2) (layer "F.Cu") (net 7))
 (segment (start 114.785 64.515) (end 114.785 65.515) (width 0.2) (layer "F.Cu") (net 7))
 (segment (start 137.984 63.499) (end 138.135 63.65) (width 0.2) (layer "F.Cu") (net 7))
 (segment (start 122.135 65.65) (end 122.286 65.801) (width 0.2) (layer "F.Cu") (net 7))
 (segment (start 121.984 63.499) (end 122.135 63.65) (width 0.2) (layer "F.Cu") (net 7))
 (segment (start 130.286 65.801) (end 132.287 65.801) (width 0.2) (layer "F.Cu") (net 7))
 (segment (start 109.91 46.23) (end 110.91 46.23) (width 0.2) (layer "F.Cu") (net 21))
 (segment (start 108.37 46.23) (end 109.37 46.23) (width 0.2) (layer "F.Cu") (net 21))
 (segment (start 109.37 46.23) (end 109.91 46.23) (width 0.2) (layer "F.Cu") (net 21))
 (segment (start 136.92 54) (end 136.44 54) (width 0.2) (layer "F.Cu") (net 8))
 (segment (start 136.44 54) (end 136.32 54) (width 0.2) (layer "F.Cu") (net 8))
 (segment (start 128.69 49.77) (end 128.69 52.845) (width 0.2) (layer "F.Cu") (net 8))
 (segment (start 126.533 55.907) (end 126.533 59.209) (width 0.2) (layer "F.Cu") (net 8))
 (segment (start 111.619 58.43) (end 116.284 63.095) (width 0.2) (layer "F.Cu") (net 8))
 (segment (start 123.405 63.401) (end 123.099 63.095) (width 0.2) (layer "F.Cu") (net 8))
 (segment (start 116.055 64.515) (end 116.055 63.515) (width 0.2) (layer "F.Cu") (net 8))
 (segment (start 123.405 63.65) (end 123.405 63.401) (width 0.2) (layer "F.Cu") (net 8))
 (segment (start 139.405 64.65) (end 139.405 63.65) (width 0.2) (layer "F.Cu") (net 8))
 (segment (start 126.533 59.209) (end 123.405 62.337) (width 0.2) (layer "F.Cu") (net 8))
 (segment (start 128.69 48.77) (end 128.69 49.77) (width 0.2) (layer "F.Cu") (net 8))
 (segment (start 131.405 64.65) (end 131.405 63.65) (width 0.2) (layer "F.Cu") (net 8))
 (segment (start 128.92 53.21) (end 128.69 52.98) (width 0.2) (layer "F.Cu") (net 8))
 (segment (start 121.285 52.845) (end 128.69 52.845) (width 0.2) (layer "F.Cu") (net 8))
 (segment (start 139.405 63.65) (end 139.405 63.074) (width 0.2) (layer "F.Cu") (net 8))
 (segment (start 131.405 63.65) (end 131.405 59.209) (width 0.2) (layer "F.Cu") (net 8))
 (segment (start 120.92 54) (end 120.92 53.21) (width 0.2) (layer "F.Cu") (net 8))
 (segment (start 116.055 63.515) (end 116.284 63.286) (width 0.2) (layer "F.Cu") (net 8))
 (segment (start 128.92 54) (end 128.44 54) (width 0.2) (layer "F.Cu") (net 8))
 (segment (start 128.92 54) (end 128.92 53.21) (width 0.2) (layer "F.Cu") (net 8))
 (segment (start 123.099 63.095) (end 116.284 63.095) (width 0.2) (layer "F.Cu") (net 8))
 (segment (start 120.92 53.21) (end 121.285 52.845) (width 0.2) (layer "F.Cu") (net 8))
 (segment (start 123.405 62.337) (end 123.405 63.401) (width 0.2) (layer "F.Cu") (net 8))
 (segment (start 112.94 53.87) (end 111.619 55.191) (width 0.2) (layer "F.Cu") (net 8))
 (segment (start 126.533 59.209) (end 131.405 59.209) (width 0.2) (layer "F.Cu") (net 8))
 (segment (start 139.405 63.074) (end 133.325 56.995) (width 0.2) (layer "F.Cu") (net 8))
 (segment (start 123.405 64.65) (end 123.405 63.65) (width 0.2) (layer "F.Cu") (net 8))
 (segment (start 113.42 53.87) (end 112.94 53.87) (width 0.2) (layer "F.Cu") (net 8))
 (segment (start 128.69 52.98) (end 128.69 52.845) (width 0.2) (layer "F.Cu") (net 8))
 (segment (start 133.325 57.289) (end 133.325 56.995) (width 0.2) (layer "F.Cu") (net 8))
 (segment (start 131.405 59.209) (end 133.325 57.289) (width 0.2) (layer "F.Cu") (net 8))
 (segment (start 136.32 54) (end 133.325 56.995) (width 0.2) (layer "F.Cu") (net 8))
 (segment (start 116.284 63.286) (end 116.284 63.095) (width 0.2) (layer "F.Cu") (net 8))
 (segment (start 111.619 55.191) (end 111.619 58.43) (width 0.2) (layer "F.Cu") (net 8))
 (segment (start 128.44 54) (end 126.533 55.907) (width 0.2) (layer "F.Cu") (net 8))
 (segment (start 108.521 49.921) (end 108.37 49.77) (width 0.2) (layer "B.Cu") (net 8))
 (segment (start 108.37 49.77) (end 108.37 48.77) (width 0.2) (layer "B.Cu") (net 8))
 (segment (start 127.539 49.921) (end 108.521 49.921) (width 0.2) (layer "B.Cu") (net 8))
 (segment (start 128.69 48.77) (end 127.983 49.477) (width 0.2) (layer "B.Cu") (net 8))
 (segment (start 127.983 49.477) (end 127.539 49.921) (width 0.2) (layer "B.Cu") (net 8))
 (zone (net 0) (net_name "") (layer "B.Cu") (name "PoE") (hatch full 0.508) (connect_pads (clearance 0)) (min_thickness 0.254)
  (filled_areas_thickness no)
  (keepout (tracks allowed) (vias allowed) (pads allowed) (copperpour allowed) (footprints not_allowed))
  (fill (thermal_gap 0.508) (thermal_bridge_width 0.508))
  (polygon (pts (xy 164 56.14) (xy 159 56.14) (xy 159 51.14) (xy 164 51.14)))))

